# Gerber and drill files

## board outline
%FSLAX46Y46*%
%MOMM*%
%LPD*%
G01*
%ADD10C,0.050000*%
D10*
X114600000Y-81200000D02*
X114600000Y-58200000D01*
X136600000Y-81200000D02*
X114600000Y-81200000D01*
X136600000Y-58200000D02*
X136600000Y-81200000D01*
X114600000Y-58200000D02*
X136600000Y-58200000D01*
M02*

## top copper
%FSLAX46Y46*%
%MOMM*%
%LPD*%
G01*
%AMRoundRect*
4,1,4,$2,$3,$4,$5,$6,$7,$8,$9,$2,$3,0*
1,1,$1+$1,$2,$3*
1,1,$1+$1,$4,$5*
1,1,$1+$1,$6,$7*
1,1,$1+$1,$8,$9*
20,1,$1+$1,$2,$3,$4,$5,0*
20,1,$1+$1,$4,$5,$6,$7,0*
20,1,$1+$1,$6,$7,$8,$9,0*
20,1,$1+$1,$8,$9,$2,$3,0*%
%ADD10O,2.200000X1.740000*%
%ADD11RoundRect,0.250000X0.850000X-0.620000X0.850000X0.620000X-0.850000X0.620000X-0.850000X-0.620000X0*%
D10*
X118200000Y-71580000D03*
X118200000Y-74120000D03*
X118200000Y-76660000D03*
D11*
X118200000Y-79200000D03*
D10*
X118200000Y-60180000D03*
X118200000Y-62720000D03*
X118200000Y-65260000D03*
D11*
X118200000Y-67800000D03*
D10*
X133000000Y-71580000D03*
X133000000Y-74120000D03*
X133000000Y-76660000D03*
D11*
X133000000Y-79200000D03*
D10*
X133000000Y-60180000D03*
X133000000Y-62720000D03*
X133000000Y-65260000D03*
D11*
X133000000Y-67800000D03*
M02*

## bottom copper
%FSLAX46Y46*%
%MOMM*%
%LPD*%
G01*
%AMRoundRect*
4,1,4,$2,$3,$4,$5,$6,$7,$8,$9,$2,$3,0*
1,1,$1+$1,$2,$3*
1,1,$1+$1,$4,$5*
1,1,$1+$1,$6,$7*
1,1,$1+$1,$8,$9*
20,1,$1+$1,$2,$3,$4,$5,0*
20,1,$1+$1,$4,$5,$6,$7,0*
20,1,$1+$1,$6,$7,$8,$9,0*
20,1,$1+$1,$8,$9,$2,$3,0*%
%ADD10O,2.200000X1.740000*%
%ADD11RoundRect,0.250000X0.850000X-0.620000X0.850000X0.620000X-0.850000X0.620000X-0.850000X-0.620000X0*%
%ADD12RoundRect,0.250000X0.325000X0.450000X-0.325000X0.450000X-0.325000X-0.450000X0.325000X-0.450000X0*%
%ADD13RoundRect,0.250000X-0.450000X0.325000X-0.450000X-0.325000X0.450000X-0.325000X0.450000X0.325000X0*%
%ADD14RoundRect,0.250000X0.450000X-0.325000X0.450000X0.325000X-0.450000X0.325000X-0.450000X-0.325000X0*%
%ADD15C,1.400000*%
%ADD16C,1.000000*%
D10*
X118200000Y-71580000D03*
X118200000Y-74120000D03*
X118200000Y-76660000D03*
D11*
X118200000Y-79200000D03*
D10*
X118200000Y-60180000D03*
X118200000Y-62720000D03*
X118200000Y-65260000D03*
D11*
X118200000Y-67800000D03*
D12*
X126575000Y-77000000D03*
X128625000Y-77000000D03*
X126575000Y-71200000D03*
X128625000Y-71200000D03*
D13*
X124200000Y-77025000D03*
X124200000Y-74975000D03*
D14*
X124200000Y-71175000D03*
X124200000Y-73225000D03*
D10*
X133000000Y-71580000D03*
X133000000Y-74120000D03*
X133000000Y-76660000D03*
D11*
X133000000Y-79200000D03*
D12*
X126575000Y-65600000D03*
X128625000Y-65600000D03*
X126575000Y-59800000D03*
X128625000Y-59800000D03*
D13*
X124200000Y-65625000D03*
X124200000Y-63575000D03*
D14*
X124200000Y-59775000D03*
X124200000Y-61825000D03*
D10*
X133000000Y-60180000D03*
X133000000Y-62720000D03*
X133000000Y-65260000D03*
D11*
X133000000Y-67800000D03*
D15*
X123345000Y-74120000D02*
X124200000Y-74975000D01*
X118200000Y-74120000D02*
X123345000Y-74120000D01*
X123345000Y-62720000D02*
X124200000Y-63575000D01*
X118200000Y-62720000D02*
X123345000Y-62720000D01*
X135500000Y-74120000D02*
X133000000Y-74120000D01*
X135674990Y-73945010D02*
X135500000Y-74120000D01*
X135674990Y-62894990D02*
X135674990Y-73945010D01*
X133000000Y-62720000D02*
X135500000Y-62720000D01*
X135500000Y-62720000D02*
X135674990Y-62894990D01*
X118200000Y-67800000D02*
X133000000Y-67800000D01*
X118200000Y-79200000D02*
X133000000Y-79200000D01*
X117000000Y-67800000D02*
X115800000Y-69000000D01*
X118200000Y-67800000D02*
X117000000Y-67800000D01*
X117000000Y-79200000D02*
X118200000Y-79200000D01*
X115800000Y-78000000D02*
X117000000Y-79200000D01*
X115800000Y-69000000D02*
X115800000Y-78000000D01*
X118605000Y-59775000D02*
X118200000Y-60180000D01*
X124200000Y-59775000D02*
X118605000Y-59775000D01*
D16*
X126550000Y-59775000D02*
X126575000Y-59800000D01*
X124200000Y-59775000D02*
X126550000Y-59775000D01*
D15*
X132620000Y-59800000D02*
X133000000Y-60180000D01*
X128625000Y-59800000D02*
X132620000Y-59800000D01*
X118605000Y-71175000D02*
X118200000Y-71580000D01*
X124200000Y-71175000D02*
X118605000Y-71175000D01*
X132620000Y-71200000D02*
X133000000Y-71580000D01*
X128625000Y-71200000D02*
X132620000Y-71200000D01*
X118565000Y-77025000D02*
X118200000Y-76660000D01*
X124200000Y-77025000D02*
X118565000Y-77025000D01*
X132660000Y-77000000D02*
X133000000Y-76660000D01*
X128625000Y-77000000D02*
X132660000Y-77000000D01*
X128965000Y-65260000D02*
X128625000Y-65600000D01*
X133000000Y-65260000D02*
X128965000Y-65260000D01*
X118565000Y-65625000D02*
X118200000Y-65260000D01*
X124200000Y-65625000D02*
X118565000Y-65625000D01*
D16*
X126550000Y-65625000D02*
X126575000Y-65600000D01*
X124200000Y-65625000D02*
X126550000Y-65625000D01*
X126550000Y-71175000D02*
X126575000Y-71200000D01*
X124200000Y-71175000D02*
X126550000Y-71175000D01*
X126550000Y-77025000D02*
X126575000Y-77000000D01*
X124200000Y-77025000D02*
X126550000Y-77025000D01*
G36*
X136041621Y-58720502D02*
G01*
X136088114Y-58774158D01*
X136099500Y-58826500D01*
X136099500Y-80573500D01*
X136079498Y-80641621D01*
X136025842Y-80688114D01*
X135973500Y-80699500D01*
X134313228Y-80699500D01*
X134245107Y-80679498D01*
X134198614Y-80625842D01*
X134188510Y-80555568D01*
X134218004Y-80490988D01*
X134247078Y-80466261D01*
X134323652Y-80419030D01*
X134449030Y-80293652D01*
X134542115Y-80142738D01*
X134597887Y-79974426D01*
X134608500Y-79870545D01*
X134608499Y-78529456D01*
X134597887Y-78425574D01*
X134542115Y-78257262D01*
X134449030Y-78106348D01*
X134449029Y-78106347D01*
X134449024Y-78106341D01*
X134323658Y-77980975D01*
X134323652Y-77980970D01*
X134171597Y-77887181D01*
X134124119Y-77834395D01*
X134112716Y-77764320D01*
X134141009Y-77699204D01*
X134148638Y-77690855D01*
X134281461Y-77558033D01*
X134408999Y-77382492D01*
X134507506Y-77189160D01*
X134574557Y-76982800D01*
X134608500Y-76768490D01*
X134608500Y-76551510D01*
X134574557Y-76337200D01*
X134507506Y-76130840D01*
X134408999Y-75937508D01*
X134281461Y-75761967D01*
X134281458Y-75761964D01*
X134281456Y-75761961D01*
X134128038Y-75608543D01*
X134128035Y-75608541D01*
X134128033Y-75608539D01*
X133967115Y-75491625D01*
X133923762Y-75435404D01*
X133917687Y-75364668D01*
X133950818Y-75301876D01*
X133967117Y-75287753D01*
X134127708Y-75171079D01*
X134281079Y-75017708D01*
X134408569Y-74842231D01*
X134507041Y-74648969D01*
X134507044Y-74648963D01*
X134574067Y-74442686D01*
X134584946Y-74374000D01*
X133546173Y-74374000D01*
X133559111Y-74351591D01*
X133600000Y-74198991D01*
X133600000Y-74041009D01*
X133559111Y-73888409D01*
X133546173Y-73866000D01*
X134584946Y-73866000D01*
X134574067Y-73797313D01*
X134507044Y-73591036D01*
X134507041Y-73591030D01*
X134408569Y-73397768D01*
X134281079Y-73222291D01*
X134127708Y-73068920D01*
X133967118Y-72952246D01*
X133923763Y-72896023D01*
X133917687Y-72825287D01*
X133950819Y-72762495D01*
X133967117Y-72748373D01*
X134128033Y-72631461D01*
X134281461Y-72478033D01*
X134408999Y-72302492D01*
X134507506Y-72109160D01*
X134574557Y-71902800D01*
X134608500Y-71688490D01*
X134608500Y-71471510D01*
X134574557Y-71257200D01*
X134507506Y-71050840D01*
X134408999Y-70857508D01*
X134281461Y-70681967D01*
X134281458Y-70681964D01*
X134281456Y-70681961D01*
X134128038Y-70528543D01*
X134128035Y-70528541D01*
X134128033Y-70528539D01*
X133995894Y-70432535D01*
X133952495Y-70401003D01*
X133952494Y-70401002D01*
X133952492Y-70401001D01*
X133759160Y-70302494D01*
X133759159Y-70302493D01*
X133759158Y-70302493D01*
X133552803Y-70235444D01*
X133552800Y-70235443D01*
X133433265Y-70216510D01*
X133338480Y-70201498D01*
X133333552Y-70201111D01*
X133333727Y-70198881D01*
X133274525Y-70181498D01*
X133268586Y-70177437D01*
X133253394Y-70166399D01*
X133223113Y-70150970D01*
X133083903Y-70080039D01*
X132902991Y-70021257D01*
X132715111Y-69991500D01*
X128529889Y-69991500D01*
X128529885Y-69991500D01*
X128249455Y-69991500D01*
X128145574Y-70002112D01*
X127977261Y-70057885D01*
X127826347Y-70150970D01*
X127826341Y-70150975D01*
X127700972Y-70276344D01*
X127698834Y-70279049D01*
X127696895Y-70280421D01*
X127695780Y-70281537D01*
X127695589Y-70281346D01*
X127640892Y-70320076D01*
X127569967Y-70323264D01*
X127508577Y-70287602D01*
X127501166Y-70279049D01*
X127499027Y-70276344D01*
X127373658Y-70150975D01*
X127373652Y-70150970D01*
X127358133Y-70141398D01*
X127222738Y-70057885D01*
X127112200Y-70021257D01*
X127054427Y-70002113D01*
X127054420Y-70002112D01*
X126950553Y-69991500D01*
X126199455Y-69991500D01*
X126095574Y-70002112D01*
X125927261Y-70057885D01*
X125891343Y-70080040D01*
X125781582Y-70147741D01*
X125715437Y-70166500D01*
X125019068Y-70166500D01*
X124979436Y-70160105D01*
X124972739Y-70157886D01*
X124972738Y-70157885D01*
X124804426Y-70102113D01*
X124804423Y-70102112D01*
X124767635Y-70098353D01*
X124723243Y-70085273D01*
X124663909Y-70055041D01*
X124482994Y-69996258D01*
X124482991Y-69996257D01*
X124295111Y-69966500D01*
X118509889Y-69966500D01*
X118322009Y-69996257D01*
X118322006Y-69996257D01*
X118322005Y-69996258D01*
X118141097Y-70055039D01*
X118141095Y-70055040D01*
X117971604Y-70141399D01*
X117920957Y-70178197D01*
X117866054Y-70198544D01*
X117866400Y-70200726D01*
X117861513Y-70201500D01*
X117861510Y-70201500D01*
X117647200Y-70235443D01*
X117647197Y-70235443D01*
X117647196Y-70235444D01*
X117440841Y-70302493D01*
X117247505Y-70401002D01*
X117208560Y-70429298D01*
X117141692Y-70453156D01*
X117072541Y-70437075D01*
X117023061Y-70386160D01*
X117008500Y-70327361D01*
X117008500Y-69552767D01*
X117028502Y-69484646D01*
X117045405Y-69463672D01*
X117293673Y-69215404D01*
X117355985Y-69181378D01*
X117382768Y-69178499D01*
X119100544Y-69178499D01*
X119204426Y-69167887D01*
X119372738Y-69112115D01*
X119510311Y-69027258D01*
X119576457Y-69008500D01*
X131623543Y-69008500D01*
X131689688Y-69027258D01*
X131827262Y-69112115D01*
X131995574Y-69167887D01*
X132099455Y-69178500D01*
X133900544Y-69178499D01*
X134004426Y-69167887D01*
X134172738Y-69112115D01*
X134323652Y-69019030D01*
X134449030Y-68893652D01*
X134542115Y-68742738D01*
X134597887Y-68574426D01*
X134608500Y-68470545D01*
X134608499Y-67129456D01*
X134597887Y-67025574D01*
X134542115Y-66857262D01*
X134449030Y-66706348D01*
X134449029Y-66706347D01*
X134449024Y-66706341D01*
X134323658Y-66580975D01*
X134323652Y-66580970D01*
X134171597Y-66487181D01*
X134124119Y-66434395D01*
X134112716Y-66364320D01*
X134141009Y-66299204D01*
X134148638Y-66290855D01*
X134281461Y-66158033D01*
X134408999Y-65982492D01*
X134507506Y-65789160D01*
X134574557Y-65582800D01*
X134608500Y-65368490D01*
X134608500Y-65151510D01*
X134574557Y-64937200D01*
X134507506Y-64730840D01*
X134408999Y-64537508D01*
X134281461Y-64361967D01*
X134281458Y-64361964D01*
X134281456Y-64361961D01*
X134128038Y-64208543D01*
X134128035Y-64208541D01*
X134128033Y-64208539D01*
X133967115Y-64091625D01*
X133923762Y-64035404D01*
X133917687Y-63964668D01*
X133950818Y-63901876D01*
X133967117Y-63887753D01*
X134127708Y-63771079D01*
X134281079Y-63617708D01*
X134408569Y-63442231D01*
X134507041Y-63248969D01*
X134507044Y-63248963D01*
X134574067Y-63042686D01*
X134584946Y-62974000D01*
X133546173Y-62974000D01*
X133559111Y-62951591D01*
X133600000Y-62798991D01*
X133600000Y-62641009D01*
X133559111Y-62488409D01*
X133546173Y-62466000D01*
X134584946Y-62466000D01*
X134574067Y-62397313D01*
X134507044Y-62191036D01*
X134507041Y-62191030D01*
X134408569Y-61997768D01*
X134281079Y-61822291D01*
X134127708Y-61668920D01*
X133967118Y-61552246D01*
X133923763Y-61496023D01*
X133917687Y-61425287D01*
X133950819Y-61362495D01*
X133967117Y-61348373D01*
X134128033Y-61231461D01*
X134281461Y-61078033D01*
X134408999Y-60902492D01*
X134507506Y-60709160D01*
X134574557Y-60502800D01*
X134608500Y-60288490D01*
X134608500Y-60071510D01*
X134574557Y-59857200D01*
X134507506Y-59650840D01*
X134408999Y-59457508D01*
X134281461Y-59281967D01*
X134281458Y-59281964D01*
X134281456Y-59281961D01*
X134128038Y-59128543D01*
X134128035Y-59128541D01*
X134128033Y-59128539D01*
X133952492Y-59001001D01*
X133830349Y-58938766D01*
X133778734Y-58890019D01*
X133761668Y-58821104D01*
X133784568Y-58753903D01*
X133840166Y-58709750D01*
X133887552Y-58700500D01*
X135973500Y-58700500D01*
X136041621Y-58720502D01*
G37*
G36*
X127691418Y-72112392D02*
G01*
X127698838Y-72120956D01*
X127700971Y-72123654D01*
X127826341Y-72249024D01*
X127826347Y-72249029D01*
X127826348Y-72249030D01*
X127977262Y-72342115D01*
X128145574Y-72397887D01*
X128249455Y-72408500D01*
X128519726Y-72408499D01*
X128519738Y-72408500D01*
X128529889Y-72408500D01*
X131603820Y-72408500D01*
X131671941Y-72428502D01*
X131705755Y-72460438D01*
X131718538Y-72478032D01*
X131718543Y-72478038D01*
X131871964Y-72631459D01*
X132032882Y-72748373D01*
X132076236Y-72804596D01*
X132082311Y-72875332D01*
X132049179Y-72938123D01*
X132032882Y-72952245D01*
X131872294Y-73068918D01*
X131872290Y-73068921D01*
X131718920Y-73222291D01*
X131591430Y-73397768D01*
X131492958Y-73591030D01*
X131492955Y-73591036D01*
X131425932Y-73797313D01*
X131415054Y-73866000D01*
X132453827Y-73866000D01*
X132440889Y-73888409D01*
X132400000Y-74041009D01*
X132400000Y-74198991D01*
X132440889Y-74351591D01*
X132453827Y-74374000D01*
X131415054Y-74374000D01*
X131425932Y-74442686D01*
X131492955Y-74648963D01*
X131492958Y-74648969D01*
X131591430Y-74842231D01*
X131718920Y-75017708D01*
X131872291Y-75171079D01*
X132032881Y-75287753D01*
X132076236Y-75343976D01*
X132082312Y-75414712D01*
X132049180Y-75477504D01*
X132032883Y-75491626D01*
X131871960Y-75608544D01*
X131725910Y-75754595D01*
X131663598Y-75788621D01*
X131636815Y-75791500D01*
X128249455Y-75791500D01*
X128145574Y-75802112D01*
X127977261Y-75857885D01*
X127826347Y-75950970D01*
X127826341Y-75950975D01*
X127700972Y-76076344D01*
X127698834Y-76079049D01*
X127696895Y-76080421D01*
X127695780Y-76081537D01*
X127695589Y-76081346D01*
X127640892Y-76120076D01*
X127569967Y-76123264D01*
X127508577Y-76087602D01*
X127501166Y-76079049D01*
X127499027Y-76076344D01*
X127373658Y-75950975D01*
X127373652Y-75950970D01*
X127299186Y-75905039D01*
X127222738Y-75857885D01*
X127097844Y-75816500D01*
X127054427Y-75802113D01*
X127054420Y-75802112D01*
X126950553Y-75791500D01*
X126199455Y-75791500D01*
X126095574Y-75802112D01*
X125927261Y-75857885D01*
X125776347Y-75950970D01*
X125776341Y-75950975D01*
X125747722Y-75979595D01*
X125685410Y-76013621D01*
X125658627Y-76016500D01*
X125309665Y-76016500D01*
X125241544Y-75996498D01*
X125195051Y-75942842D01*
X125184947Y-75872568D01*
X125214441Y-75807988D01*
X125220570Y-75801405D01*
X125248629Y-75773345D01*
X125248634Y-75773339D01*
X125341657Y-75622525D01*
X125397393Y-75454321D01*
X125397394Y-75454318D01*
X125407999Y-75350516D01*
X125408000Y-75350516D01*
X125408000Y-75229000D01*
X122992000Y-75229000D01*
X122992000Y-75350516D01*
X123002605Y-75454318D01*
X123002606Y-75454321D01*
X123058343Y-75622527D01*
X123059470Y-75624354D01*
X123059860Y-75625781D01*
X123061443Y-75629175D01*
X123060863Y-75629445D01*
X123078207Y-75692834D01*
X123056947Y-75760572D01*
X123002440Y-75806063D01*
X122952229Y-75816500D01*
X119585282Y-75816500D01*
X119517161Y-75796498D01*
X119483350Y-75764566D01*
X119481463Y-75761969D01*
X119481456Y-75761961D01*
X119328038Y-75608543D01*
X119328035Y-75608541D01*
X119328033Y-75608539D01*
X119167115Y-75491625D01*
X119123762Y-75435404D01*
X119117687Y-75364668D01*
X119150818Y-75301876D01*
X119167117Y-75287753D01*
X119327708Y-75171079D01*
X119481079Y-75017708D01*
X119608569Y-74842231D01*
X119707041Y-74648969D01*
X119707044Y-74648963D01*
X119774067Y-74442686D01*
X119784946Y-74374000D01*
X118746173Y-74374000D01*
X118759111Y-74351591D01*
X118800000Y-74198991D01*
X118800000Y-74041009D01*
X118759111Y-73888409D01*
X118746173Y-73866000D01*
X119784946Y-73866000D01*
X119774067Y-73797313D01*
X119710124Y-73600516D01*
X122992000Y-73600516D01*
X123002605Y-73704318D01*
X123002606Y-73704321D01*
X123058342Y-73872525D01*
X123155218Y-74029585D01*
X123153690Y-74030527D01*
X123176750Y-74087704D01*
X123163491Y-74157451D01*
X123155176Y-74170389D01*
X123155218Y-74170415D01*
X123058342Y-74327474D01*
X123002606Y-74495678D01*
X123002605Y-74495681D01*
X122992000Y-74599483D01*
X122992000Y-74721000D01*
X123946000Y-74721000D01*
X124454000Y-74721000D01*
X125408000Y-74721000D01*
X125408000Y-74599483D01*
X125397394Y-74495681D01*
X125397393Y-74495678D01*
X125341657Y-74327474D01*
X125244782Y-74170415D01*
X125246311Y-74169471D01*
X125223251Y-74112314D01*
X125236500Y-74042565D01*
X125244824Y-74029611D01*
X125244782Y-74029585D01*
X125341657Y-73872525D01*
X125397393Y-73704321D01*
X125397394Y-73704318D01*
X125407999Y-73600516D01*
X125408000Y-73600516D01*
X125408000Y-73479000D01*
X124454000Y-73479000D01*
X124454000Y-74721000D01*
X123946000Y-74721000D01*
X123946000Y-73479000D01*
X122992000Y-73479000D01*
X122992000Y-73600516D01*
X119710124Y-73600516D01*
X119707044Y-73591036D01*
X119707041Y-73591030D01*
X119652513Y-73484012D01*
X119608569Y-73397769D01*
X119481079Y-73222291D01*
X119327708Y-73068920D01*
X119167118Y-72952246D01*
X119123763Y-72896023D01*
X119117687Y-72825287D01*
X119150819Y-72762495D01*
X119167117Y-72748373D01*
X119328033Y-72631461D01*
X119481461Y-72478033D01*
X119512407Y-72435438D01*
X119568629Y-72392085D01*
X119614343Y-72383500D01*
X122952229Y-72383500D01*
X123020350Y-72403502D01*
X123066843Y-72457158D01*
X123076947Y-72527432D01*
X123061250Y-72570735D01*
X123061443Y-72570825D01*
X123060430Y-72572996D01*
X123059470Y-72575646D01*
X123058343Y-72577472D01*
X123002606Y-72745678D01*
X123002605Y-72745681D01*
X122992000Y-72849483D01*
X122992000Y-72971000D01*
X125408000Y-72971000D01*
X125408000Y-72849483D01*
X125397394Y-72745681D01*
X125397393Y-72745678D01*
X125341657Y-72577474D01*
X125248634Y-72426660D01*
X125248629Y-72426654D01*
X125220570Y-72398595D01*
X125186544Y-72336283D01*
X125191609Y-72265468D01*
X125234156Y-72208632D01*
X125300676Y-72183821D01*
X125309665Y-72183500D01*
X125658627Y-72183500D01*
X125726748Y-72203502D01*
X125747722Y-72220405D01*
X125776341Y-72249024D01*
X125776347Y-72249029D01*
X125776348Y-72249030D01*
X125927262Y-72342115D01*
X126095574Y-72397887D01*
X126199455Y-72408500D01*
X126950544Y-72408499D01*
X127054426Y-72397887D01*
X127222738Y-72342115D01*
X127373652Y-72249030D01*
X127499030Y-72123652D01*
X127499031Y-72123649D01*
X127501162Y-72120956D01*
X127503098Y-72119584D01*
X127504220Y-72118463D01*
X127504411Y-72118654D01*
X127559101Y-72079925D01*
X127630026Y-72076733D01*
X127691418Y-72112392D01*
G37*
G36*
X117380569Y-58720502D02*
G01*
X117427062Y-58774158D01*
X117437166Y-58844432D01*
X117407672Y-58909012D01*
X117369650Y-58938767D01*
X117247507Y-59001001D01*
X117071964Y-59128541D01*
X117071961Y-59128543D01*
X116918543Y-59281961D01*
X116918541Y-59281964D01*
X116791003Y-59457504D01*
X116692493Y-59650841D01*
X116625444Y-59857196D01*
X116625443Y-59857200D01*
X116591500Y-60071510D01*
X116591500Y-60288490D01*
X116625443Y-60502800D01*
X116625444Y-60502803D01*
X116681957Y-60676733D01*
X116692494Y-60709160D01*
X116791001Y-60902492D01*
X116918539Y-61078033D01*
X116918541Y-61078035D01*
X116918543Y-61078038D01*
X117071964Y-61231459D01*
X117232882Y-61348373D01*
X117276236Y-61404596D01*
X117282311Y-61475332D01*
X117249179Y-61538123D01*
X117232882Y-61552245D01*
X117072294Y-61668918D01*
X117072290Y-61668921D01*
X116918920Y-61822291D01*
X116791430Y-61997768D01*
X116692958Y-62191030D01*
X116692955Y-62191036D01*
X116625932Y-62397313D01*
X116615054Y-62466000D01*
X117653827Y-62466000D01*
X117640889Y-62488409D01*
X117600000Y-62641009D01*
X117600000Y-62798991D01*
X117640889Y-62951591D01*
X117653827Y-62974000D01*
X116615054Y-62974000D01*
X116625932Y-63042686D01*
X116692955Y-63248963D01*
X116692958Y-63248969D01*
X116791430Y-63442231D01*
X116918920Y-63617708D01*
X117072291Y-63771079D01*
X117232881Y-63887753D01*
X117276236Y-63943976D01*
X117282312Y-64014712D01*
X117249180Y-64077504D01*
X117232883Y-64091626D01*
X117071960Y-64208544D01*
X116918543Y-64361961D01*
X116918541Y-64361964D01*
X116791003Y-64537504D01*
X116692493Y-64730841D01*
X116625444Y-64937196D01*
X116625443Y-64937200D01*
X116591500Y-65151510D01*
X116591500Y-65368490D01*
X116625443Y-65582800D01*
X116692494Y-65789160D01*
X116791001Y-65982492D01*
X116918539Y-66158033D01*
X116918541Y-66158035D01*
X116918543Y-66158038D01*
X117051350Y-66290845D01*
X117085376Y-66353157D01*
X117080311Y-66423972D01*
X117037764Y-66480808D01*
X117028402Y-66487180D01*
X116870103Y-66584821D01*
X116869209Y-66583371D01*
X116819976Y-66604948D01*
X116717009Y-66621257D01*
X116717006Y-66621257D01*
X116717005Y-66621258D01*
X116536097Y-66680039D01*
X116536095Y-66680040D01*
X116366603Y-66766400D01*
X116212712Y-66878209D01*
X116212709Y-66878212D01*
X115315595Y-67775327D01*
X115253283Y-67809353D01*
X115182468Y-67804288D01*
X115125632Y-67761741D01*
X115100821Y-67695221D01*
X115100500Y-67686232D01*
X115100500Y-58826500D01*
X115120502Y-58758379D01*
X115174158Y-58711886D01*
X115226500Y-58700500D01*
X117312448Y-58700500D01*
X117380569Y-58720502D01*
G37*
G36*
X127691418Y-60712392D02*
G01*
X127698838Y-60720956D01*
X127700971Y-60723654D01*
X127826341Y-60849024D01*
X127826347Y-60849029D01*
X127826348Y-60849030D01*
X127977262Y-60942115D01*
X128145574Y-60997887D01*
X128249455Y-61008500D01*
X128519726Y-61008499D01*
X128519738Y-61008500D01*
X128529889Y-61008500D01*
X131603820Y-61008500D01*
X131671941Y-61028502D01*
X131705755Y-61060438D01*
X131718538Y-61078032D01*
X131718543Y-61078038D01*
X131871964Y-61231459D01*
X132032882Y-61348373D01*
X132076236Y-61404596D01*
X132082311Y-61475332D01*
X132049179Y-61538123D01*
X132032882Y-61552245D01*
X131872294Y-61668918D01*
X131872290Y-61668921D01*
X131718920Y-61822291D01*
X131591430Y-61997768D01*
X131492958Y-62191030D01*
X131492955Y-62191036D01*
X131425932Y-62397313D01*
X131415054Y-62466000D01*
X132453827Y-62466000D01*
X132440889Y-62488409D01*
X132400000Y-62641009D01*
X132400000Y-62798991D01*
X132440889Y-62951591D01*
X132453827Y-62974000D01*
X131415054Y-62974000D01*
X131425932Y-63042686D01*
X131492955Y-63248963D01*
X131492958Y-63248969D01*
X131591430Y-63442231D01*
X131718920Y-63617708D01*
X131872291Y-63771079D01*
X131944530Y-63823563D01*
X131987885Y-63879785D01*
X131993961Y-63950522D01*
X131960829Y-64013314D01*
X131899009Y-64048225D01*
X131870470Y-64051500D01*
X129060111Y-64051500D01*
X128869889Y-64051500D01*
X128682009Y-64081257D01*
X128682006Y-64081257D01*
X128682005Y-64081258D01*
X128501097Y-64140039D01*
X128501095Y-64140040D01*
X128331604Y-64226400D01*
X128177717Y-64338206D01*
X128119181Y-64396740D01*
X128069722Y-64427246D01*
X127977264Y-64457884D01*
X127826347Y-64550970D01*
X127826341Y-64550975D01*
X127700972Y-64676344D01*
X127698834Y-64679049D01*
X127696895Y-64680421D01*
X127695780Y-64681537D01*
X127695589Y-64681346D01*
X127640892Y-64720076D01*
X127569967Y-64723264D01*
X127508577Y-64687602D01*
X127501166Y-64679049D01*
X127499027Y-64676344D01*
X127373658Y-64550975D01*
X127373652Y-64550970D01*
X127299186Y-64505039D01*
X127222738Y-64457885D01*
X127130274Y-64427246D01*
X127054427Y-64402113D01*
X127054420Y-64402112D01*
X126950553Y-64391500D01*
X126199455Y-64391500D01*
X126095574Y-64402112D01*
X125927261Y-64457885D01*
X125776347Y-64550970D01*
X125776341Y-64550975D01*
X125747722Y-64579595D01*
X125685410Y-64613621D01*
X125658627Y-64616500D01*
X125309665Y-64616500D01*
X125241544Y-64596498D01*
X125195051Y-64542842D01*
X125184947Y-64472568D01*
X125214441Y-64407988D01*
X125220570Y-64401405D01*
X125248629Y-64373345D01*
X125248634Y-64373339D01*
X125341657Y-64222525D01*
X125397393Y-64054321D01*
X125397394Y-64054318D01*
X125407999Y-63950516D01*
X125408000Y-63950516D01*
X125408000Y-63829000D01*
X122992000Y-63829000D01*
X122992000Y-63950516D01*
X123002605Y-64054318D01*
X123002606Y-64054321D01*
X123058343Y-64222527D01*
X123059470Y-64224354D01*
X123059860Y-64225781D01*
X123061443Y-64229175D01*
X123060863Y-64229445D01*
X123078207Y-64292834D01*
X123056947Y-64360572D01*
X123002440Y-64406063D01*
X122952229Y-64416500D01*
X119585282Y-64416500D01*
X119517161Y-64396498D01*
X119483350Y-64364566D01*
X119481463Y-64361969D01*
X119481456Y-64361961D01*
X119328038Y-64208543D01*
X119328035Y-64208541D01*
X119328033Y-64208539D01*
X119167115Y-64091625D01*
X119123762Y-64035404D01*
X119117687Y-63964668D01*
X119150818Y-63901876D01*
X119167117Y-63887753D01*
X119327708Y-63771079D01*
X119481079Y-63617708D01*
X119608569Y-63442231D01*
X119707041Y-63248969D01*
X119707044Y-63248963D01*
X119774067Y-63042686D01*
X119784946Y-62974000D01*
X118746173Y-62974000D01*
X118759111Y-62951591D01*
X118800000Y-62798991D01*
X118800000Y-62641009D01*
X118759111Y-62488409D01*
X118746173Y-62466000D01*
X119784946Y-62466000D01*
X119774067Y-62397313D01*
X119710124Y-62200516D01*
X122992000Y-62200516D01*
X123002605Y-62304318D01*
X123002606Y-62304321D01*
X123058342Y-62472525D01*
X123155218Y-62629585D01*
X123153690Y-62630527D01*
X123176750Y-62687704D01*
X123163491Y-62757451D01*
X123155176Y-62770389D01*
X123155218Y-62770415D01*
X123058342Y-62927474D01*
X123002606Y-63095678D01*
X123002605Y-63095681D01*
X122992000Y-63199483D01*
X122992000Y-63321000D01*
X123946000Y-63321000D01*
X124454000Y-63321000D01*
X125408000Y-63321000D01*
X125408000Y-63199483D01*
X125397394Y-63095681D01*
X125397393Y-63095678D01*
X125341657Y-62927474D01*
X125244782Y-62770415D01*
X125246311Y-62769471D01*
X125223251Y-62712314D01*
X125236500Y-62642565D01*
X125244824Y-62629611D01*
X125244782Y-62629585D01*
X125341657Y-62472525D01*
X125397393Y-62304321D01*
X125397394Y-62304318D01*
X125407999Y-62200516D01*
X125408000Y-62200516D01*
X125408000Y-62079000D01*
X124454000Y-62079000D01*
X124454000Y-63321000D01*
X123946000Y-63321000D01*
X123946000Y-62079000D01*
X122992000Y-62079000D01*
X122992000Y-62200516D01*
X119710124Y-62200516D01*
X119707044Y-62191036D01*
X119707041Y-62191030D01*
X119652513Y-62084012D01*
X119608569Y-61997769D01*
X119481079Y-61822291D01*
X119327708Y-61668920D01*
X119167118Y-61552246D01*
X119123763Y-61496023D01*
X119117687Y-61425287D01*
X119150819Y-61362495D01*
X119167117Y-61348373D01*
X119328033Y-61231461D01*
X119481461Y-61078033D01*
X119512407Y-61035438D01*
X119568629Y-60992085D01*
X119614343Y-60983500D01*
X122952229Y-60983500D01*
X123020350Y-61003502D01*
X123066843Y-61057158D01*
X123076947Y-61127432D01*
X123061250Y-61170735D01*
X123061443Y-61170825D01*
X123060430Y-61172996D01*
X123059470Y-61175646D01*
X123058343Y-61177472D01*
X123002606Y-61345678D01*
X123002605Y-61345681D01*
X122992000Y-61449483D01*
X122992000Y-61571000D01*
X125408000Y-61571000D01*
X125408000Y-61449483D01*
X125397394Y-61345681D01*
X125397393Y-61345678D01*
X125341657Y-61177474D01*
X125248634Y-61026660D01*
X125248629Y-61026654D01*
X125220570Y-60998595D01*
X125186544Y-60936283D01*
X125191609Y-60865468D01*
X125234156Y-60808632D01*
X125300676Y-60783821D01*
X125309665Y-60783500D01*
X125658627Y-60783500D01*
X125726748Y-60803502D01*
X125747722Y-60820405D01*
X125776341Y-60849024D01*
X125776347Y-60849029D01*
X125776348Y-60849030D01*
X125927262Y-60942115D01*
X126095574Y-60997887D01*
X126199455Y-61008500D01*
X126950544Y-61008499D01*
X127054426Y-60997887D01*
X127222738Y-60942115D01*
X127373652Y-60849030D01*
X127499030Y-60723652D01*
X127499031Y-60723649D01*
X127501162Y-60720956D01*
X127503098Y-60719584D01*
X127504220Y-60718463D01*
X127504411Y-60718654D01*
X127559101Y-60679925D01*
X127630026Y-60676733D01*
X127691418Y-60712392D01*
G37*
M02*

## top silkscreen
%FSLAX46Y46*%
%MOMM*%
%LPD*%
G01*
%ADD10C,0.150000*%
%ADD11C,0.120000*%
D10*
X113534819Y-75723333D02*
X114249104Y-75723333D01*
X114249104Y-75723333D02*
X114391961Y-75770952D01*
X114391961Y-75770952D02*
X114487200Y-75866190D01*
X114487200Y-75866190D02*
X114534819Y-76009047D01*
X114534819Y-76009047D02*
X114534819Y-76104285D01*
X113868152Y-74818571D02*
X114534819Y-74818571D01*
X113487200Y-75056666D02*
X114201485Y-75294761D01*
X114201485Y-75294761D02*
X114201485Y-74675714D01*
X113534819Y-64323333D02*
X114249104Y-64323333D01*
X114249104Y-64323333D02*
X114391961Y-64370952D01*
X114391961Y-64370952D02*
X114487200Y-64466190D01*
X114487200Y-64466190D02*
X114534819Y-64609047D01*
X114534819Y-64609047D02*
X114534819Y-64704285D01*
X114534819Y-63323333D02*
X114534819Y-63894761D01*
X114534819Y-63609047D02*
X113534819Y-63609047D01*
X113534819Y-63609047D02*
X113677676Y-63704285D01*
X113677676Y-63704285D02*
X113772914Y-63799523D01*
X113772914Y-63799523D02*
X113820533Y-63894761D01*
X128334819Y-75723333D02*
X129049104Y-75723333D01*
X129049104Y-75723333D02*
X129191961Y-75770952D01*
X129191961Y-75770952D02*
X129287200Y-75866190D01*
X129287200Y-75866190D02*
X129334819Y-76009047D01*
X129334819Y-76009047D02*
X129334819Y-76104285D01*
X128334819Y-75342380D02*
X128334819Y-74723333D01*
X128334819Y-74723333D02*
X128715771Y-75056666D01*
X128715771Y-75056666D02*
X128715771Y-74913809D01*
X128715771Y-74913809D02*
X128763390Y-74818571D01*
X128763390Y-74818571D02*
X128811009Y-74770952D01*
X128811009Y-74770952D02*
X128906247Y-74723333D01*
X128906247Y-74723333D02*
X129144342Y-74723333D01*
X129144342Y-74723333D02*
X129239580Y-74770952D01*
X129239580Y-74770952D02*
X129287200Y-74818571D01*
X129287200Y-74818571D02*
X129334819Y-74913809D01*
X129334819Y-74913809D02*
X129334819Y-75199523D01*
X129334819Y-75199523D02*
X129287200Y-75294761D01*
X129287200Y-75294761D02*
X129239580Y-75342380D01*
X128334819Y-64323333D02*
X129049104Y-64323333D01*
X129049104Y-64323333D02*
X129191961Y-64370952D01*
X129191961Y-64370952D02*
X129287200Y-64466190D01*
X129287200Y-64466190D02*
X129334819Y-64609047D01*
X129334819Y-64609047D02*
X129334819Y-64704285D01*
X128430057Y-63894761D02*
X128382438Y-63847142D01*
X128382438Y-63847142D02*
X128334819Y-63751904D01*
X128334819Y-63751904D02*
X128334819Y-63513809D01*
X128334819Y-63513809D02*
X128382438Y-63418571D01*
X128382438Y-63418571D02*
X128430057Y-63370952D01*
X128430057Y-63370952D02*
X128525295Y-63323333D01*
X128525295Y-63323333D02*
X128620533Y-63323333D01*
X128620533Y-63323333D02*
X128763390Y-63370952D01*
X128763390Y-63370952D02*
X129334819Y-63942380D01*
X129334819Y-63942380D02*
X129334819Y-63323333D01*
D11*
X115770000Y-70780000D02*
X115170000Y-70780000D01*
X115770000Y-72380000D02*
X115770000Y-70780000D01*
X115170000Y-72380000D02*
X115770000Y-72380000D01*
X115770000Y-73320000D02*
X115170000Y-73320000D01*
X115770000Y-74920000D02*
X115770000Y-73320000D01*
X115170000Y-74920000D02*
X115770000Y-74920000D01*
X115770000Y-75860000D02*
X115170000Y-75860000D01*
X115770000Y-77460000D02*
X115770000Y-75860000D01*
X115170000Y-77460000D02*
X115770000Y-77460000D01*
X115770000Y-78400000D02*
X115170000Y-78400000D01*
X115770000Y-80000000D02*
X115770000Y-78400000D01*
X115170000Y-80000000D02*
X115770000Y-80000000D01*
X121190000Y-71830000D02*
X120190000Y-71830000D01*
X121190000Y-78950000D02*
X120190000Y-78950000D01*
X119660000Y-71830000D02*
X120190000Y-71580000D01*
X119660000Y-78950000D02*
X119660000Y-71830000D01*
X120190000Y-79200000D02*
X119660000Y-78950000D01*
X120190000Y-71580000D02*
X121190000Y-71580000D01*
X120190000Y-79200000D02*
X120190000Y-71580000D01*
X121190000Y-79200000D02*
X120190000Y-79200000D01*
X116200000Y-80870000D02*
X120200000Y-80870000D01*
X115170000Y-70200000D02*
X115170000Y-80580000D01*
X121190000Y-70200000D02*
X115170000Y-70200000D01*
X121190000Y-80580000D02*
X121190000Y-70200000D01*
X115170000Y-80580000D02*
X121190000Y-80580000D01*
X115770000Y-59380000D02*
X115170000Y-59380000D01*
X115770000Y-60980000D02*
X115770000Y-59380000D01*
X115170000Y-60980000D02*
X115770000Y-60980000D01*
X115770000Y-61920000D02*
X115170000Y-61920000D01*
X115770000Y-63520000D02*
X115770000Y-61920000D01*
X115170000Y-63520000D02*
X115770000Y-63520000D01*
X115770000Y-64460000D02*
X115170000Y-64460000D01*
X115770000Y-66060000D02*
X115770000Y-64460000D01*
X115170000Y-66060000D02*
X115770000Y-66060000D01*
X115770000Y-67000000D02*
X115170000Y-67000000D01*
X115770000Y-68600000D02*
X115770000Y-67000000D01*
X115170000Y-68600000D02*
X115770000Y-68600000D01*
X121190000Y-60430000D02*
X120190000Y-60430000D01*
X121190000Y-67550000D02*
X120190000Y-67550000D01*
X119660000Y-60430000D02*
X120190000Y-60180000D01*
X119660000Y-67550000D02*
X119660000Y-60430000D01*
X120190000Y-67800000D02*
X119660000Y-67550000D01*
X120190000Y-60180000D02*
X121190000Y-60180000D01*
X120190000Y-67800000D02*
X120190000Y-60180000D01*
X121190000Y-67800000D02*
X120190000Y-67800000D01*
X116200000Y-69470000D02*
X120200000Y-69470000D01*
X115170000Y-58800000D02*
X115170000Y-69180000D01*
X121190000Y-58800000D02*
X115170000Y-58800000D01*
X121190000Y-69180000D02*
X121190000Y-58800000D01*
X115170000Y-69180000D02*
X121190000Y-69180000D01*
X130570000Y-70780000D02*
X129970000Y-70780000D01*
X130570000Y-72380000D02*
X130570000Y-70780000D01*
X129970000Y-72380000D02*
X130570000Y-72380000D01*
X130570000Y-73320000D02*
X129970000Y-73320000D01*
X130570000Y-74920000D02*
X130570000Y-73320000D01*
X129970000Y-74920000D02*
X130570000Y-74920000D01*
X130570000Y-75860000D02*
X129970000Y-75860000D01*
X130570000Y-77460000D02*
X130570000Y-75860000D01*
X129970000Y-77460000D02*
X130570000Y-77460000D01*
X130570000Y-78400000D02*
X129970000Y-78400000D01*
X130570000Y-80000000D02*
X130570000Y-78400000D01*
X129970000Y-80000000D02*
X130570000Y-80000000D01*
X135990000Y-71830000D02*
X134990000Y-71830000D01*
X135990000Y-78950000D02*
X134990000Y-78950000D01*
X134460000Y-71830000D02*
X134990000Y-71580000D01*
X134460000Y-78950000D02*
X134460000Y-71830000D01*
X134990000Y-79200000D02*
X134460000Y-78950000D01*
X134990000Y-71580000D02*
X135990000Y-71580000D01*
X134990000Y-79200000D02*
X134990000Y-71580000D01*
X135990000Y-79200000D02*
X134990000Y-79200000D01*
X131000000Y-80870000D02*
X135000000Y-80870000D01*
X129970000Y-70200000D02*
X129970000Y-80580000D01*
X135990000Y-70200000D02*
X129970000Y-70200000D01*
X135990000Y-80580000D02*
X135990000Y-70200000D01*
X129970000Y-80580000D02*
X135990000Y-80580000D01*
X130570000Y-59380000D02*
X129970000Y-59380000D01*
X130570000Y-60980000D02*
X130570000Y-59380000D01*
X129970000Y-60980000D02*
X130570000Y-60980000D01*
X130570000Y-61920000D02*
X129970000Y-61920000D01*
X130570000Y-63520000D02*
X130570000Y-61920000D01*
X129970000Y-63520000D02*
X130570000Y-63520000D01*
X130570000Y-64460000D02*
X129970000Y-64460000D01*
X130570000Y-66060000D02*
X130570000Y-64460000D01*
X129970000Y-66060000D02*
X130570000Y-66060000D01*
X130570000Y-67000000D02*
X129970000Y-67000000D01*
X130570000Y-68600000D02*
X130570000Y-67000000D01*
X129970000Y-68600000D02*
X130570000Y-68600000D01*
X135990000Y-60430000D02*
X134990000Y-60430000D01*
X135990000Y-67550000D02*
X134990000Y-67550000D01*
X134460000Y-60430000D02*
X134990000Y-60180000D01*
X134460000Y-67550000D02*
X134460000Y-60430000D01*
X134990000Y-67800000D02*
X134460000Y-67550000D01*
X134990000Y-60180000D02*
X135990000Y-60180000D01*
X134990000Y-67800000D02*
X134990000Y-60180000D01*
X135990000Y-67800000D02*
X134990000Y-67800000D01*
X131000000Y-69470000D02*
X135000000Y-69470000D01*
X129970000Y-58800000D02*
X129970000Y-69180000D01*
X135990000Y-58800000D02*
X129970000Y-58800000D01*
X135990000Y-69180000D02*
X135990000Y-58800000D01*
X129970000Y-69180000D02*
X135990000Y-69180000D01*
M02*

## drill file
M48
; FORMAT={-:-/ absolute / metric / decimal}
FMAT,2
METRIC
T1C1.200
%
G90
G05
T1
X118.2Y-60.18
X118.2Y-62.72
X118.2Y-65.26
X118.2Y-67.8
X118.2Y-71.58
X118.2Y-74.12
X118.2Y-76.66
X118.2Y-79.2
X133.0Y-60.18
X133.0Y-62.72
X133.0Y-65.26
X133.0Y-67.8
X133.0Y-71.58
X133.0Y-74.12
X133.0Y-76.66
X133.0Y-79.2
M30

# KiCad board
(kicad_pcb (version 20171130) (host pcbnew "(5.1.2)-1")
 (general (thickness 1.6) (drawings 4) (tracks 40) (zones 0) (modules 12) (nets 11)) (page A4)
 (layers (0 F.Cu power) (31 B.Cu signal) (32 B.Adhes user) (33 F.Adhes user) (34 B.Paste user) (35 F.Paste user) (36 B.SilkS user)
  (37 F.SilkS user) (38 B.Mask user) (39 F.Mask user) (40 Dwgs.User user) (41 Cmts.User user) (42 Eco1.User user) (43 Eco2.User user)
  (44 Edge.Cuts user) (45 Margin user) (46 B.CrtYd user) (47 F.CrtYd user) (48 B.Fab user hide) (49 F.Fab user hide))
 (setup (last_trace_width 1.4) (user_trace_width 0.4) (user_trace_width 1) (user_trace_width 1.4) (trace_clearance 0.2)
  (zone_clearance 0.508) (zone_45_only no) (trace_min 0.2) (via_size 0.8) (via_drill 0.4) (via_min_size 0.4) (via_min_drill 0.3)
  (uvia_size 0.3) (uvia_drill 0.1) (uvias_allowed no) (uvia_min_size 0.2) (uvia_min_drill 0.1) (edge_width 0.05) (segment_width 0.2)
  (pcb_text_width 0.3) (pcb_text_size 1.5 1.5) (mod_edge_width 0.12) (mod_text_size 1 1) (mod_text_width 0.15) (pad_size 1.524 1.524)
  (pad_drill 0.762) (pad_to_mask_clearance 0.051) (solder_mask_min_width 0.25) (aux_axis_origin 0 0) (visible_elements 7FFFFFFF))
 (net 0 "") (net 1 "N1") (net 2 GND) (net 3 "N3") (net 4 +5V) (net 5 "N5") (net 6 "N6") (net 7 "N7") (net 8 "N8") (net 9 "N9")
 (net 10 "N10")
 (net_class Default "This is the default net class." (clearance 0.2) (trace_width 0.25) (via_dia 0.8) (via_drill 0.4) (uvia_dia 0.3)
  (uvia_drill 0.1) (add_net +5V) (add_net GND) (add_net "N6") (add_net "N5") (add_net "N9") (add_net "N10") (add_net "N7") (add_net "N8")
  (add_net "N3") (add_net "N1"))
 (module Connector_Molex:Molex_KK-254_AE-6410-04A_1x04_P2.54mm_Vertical (layer F.Cu) (at 118.2 79.2 90)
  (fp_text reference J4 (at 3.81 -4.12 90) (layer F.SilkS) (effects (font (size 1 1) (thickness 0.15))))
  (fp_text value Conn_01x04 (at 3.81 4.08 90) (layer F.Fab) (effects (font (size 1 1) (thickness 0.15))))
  (fp_line (start 8.42 -2.43) (end 8.42 -3.03) (layer F.SilkS) (width 0.12))
  (fp_line (start 6.82 -2.43) (end 8.42 -2.43) (layer F.SilkS) (width 0.12))
  (fp_line (start 6.82 -3.03) (end 6.82 -2.43) (layer F.SilkS) (width 0.12))
  (fp_line (start 5.88 -2.43) (end 5.88 -3.03) (layer F.SilkS) (width 0.12))
  (fp_line (start 4.28 -2.43) (end 5.88 -2.43) (layer F.SilkS) (width 0.12))
  (fp_line (start 4.28 -3.03) (end 4.28 -2.43) (layer F.SilkS) (width 0.12))
  (fp_line (start 3.34 -2.43) (end 3.34 -3.03) (layer F.SilkS) (width 0.12))
  (fp_line (start 1.74 -2.43) (end 3.34 -2.43) (layer F.SilkS) (width 0.12))
  (fp_line (start 1.74 -3.03) (end 1.74 -2.43) (layer F.SilkS) (width 0.12))
  (fp_line (start 0.8 -2.43) (end 0.8 -3.03) (layer F.SilkS) (width 0.12))
  (fp_line (start -0.8 -2.43) (end 0.8 -2.43) (layer F.SilkS) (width 0.12))
  (fp_line (start -0.8 -3.03) (end -0.8 -2.43) (layer F.SilkS) (width 0.12))
  (fp_line (start 7.37 2.99) (end 7.37 1.99) (layer F.SilkS) (width 0.12))
  (fp_line (start 0.25 2.99) (end 0.25 1.99) (layer F.SilkS) (width 0.12))
  (fp_line (start 7.37 1.46) (end 7.62 1.99) (layer F.SilkS) (width 0.12))
  (fp_line (start 0.25 1.46) (end 7.37 1.46) (layer F.SilkS) (width 0.12))
  (fp_line (start 0 1.99) (end 0.25 1.46) (layer F.SilkS) (width 0.12))
  (fp_line (start 7.62 1.99) (end 7.62 2.99) (layer F.SilkS) (width 0.12))
  (fp_line (start 0 1.99) (end 7.62 1.99) (layer F.SilkS) (width 0.12))
  (fp_line (start 0 2.99) (end 0 1.99) (layer F.SilkS) (width 0.12))
  (fp_line (start -1.67 -2) (end -1.67 2) (layer F.SilkS) (width 0.12))
  (fp_line (start 9 -3.03) (end -1.38 -3.03) (layer F.SilkS) (width 0.12))
  (fp_line (start 9 2.99) (end 9 -3.03) (layer F.SilkS) (width 0.12))
  (fp_line (start -1.38 2.99) (end 9 2.99) (layer F.SilkS) (width 0.12))
  (fp_line (start -1.38 -3.03) (end -1.38 2.99) (layer F.SilkS) (width 0.12))
  (pad 4 thru_hole oval (at 7.62 0 90) (size 1.74 2.2) (drill 1.2) (layers *.Cu *.Mask) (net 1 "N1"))
  (pad 3 thru_hole oval (at 5.08 0 90) (size 1.74 2.2) (drill 1.2) (layers *.Cu *.Mask) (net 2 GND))
  (pad 2 thru_hole oval (at 2.54 0 90) (size 1.74 2.2) (drill 1.2) (layers *.Cu *.Mask) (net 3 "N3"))
  (pad 1 thru_hole roundrect (at 0 0 90) (size 1.74 2.2) (drill 1.2) (layers *.Cu *.Mask) (roundrect_rratio 0.143678) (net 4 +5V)))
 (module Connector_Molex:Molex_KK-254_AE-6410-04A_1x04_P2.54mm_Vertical (layer F.Cu) (at 118.2 67.8 90)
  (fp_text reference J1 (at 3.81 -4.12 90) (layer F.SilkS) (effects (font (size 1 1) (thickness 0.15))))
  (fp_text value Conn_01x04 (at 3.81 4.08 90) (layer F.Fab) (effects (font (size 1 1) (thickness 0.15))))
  (fp_line (start 8.42 -2.43) (end 8.42 -3.03) (layer F.SilkS) (width 0.12))
  (fp_line (start 6.82 -2.43) (end 8.42 -2.43) (layer F.SilkS) (width 0.12))
  (fp_line (start 6.82 -3.03) (end 6.82 -2.43) (layer F.SilkS) (width 0.12))
  (fp_line (start 5.88 -2.43) (end 5.88 -3.03) (layer F.SilkS) (width 0.12))
  (fp_line (start 4.28 -2.43) (end 5.88 -2.43) (layer F.SilkS) (width 0.12))
  (fp_line (start 4.28 -3.03) (end 4.28 -2.43) (layer F.SilkS) (width 0.12))
  (fp_line (start 3.34 -2.43) (end 3.34 -3.03) (layer F.SilkS) (width 0.12))
  (fp_line (start 1.74 -2.43) (end 3.34 -2.43) (layer F.SilkS) (width 0.12))
  (fp_line (start 1.74 -3.03) (end 1.74 -2.43) (layer F.SilkS) (width 0.12))
  (fp_line (start 0.8 -2.43) (end 0.8 -3.03) (layer F.SilkS) (width 0.12))
  (fp_line (start -0.8 -2.43) (end 0.8 -2.43) (layer F.SilkS) (width 0.12))
  (fp_line (start -0.8 -3.03) (end -0.8 -2.43) (layer F.SilkS) (width 0.12))
  (fp_line (start 7.37 2.99) (end 7.37 1.99) (layer F.SilkS) (width 0.12))
  (fp_line (start 0.25 2.99) (end 0.25 1.99) (layer F.SilkS) (width 0.12))
  (fp_line (start 7.37 1.46) (end 7.62 1.99) (layer F.SilkS) (width 0.12))
  (fp_line (start 0.25 1.46) (end 7.37 1.46) (layer F.SilkS) (width 0.12))
  (fp_line (start 0 1.99) (end 0.25 1.46) (layer F.SilkS) (width 0.12))
  (fp_line (start 7.62 1.99) (end 7.62 2.99) (layer F.SilkS) (width 0.12))
  (fp_line (start 0 1.99) (end 7.62 1.99) (layer F.SilkS) (width 0.12))
  (fp_line (start 0 2.99) (end 0 1.99) (layer F.SilkS) (width 0.12))
  (fp_line (start -1.67 -2) (end -1.67 2) (layer F.SilkS) (width 0.12))
  (fp_line (start 9 -3.03) (end -1.38 -3.03) (layer F.SilkS) (width 0.12))
  (fp_line (start 9 2.99) (end 9 -3.03) (layer F.SilkS) (width 0.12))
  (fp_line (start -1.38 2.99) (end 9 2.99) (layer F.SilkS) (width 0.12))
  (fp_line (start -1.38 -3.03) (end -1.38 2.99) (layer F.SilkS) (width 0.12))
  (pad 4 thru_hole oval (at 7.62 0 90) (size 1.74 2.2) (drill 1.2) (layers *.Cu *.Mask) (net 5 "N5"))
  (pad 3 thru_hole oval (at 5.08 0 90) (size 1.74 2.2) (drill 1.2) (layers *.Cu *.Mask) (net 2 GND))
  (pad 2 thru_hole oval (at 2.54 0 90) (size 1.74 2.2) (drill 1.2) (layers *.Cu *.Mask) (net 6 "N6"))
  (pad 1 thru_hole roundrect (at 0 0 90) (size 1.74 2.2) (drill 1.2) (layers *.Cu *.Mask) (roundrect_rratio 0.143678) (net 4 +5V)))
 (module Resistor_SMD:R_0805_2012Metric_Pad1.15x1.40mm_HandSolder (layer B.Cu) (at 127.6 77 180)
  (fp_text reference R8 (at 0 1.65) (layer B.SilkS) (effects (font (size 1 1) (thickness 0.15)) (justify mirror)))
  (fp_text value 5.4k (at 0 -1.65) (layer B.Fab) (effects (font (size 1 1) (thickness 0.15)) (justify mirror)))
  (pad 2 smd roundrect (at 1.025 0 180) (size 1.15 1.4) (layers B.Cu B.Paste B.Mask) (roundrect_rratio 0.217391) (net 3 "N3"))
  (pad 1 smd roundrect (at -1.025 0 180) (size 1.15 1.4) (layers B.Cu B.Paste B.Mask) (roundrect_rratio 0.217391) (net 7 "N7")))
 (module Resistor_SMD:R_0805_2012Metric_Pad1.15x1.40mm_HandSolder (layer B.Cu) (at 127.6 71.2 180)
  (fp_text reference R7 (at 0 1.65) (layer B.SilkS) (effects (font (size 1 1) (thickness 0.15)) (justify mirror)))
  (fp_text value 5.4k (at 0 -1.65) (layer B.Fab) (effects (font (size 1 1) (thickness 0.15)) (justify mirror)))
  (pad 2 smd roundrect (at 1.025 0 180) (size 1.15 1.4) (layers B.Cu B.Paste B.Mask) (roundrect_rratio 0.217391) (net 1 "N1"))
  (pad 1 smd roundrect (at -1.025 0 180) (size 1.15 1.4) (layers B.Cu B.Paste B.Mask) (roundrect_rratio 0.217391) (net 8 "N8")))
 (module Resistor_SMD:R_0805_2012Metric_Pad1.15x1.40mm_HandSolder (layer B.Cu) (at 124.2 76 270)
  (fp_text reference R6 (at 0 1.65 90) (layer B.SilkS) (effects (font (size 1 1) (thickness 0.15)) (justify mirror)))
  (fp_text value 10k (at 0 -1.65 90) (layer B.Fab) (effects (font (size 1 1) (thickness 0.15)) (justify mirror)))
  (pad 2 smd roundrect (at 1.025 0 270) (size 1.15 1.4) (layers B.Cu B.Paste B.Mask) (roundrect_rratio 0.217391) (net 3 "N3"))
  (pad 1 smd roundrect (at -1.025 0 270) (size 1.15 1.4) (layers B.Cu B.Paste B.Mask) (roundrect_rratio 0.217391) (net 2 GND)))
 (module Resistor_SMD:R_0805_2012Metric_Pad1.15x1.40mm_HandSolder (layer B.Cu) (at 124.2 72.2 90)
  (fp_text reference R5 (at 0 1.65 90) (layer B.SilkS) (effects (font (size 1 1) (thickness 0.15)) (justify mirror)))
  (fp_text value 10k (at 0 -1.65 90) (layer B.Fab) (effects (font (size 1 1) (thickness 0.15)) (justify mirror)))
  (pad 2 smd roundrect (at 1.025 0 90) (size 1.15 1.4) (layers B.Cu B.Paste B.Mask) (roundrect_rratio 0.217391) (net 1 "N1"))
  (pad 1 smd roundrect (at -1.025 0 90) (size 1.15 1.4) (layers B.Cu B.Paste B.Mask) (roundrect_rratio 0.217391) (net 2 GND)))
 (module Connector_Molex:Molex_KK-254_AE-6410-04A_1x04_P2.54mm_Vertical (layer F.Cu) (at 133 79.2 90)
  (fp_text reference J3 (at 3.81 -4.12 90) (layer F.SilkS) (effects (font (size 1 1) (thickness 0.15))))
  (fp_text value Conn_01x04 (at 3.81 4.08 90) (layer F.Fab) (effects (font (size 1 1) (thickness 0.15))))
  (fp_line (start 8.42 -2.43) (end 8.42 -3.03) (layer F.SilkS) (width 0.12))
  (fp_line (start 6.82 -2.43) (end 8.42 -2.43) (layer F.SilkS) (width 0.12))
  (fp_line (start 6.82 -3.03) (end 6.82 -2.43) (layer F.SilkS) (width 0.12))
  (fp_line (start 5.88 -2.43) (end 5.88 -3.03) (layer F.SilkS) (width 0.12))
  (fp_line (start 4.28 -2.43) (end 5.88 -2.43) (layer F.SilkS) (width 0.12))
  (fp_line (start 4.28 -3.03) (end 4.28 -2.43) (layer F.SilkS) (width 0.12))
  (fp_line (start 3.34 -2.43) (end 3.34 -3.03) (layer F.SilkS) (width 0.12))
  (fp_line (start 1.74 -2.43) (end 3.34 -2.43) (layer F.SilkS) (width 0.12))
  (fp_line (start 1.74 -3.03) (end 1.74 -2.43) (layer F.SilkS) (width 0.12))
  (fp_line (start 0.8 -2.43) (end 0.8 -3.03) (layer F.SilkS) (width 0.12))
  (fp_line (start -0.8 -2.43) (end 0.8 -2.43) (layer F.SilkS) (width 0.12))
  (fp_line (start -0.8 -3.03) (end -0.8 -2.43) (layer F.SilkS) (width 0.12))
  (fp_line (start 7.37 2.99) (end 7.37 1.99) (layer F.SilkS) (width 0.12))
  (fp_line (start 0.25 2.99) (end 0.25 1.99) (layer F.SilkS) (width 0.12))
  (fp_line (start 7.37 1.46) (end 7.62 1.99) (layer F.SilkS) (width 0.12))
  (fp_line (start 0.25 1.46) (end 7.37 1.46) (layer F.SilkS) (width 0.12))
  (fp_line (start 0 1.99) (end 0.25 1.46) (layer F.SilkS) (width 0.12))
  (fp_line (start 7.62 1.99) (end 7.62 2.99) (layer F.SilkS) (width 0.12))
  (fp_line (start 0 1.99) (end 7.62 1.99) (layer F.SilkS) (width 0.12))
  (fp_line (start 0 2.99) (end 0 1.99) (layer F.SilkS) (width 0.12))
  (fp_line (start -1.67 -2) (end -1.67 2) (layer F.SilkS) (width 0.12))
  (fp_line (start 9 -3.03) (end -1.38 -3.03) (layer F.SilkS) (width 0.12))
  (fp_line (start 9 2.99) (end 9 -3.03) (layer F.SilkS) (width 0.12))
  (fp_line (start -1.38 2.99) (end 9 2.99) (layer F.SilkS) (width 0.12))
  (fp_line (start -1.38 -3.03) (end -1.38 2.99) (layer F.SilkS) (width 0.12))
  (pad 4 thru_hole oval (at 7.62 0 90) (size 1.74 2.2) (drill 1.2) (layers *.Cu *.Mask) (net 8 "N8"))
  (pad 3 thru_hole oval (at 5.08 0 90) (size 1.74 2.2) (drill 1.2) (layers *.Cu *.Mask) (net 2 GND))
  (pad 2 thru_hole oval (at 2.54 0 90) (size 1.74 2.2) (drill 1.2) (layers *.Cu *.Mask) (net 7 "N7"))
  (pad 1 thru_hole roundrect (at 0 0 90) (size 1.74 2.2) (drill 1.2) (layers *.Cu *.Mask) (roundrect_rratio 0.143678) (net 4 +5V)))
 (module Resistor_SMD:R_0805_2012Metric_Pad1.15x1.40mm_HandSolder (layer B.Cu) (at 127.6 65.6 180)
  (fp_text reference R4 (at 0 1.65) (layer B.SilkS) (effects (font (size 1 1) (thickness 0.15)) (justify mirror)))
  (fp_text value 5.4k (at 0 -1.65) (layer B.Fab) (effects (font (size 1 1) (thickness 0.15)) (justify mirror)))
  (pad 2 smd roundrect (at 1.025 0 180) (size 1.15 1.4) (layers B.Cu B.Paste B.Mask) (roundrect_rratio 0.217391) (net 6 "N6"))
  (pad 1 smd roundrect (at -1.025 0 180) (size 1.15 1.4) (layers B.Cu B.Paste B.Mask) (roundrect_rratio 0.217391) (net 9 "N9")))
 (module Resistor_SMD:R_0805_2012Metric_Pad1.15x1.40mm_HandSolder (layer B.Cu) (at 127.6 59.8 180)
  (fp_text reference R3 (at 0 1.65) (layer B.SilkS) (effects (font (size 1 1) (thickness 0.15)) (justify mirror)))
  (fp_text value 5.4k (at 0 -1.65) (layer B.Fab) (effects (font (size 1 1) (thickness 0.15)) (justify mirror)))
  (pad 2 smd roundrect (at 1.025 0 180) (size 1.15 1.4) (layers B.Cu B.Paste B.Mask) (roundrect_rratio 0.217391) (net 5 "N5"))
  (pad 1 smd roundrect (at -1.025 0 180) (size 1.15 1.4) (layers B.Cu B.Paste B.Mask) (roundrect_rratio 0.217391) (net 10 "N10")))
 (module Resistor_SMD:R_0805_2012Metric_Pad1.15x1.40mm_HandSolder (layer B.Cu) (at 124.2 64.6 270)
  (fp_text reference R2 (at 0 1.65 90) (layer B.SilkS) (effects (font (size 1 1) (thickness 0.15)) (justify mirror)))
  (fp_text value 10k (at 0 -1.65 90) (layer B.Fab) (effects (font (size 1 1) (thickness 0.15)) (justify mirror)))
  (pad 2 smd roundrect (at 1.025 0 270) (size 1.15 1.4) (layers B.Cu B.Paste B.Mask) (roundrect_rratio 0.217391) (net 6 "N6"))
  (pad 1 smd roundrect (at -1.025 0 270) (size 1.15 1.4) (layers B.Cu B.Paste B.Mask) (roundrect_rratio 0.217391) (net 2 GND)))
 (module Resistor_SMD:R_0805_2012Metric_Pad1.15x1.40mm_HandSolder (layer B.Cu) (at 124.2 60.8 90)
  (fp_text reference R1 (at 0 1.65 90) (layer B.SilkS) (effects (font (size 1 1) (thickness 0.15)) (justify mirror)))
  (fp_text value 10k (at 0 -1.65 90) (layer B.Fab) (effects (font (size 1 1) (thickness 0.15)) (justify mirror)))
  (pad 2 smd roundrect (at 1.025 0 90) (size 1.15 1.4) (layers B.Cu B.Paste B.Mask) (roundrect_rratio 0.217391) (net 5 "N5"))
  (pad 1 smd roundrect (at -1.025 0 90) (size 1.15 1.4) (layers B.Cu B.Paste B.Mask) (roundrect_rratio 0.217391) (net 2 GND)))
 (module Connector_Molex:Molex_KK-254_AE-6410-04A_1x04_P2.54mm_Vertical (layer F.Cu) (at 133 67.8 90)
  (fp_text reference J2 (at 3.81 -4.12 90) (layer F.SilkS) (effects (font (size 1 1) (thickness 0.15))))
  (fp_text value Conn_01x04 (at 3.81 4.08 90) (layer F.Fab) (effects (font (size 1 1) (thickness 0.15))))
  (fp_line (start 8.42 -2.43) (end 8.42 -3.03) (layer F.SilkS) (width 0.12))
  (fp_line (start 6.82 -2.43) (end 8.42 -2.43) (layer F.SilkS) (width 0.12))
  (fp_line (start 6.82 -3.03) (end 6.82 -2.43) (layer F.SilkS) (width 0.12))
  (fp_line (start 5.88 -2.43) (end 5.88 -3.03) (layer F.SilkS) (width 0.12))
  (fp_line (start 4.28 -2.43) (end 5.88 -2.43) (layer F.SilkS) (width 0.12))
  (fp_line (start 4.28 -3.03) (end 4.28 -2.43) (layer F.SilkS) (width 0.12))
  (fp_line (start 3.34 -2.43) (end 3.34 -3.03) (layer F.SilkS) (width 0.12))
  (fp_line (start 1.74 -2.43) (end 3.34 -2.43) (layer F.SilkS) (width 0.12))
  (fp_line (start 1.74 -3.03) (end 1.74 -2.43) (layer F.SilkS) (width 0.12))
  (fp_line (start 0.8 -2.43) (end 0.8 -3.03) (layer F.SilkS) (width 0.12))
  (fp_line (start -0.8 -2.43) (end 0.8 -2.43) (layer F.SilkS) (width 0.12))
  (fp_line (start -0.8 -3.03) (end -0.8 -2.43) (layer F.SilkS) (width 0.12))
  (fp_line (start 7.37 2.99) (end 7.37 1.99) (layer F.SilkS) (width 0.12))
  (fp_line (start 0.25 2.99) (end 0.25 1.99) (layer F.SilkS) (width 0.12))
  (fp_line (start 7.37 1.46) (end 7.62 1.99) (layer F.SilkS) (width 0.12))
  (fp_line (start 0.25 1.46) (end 7.37 1.46) (layer F.SilkS) (width 0.12))
  (fp_line (start 0 1.99) (end 0.25 1.46) (layer F.SilkS) (width 0.12))
  (fp_line (start 7.62 1.99) (end 7.62 2.99) (layer F.SilkS) (width 0.12))
  (fp_line (start 0 1.99) (end 7.62 1.99) (layer F.SilkS) (width 0.12))
  (fp_line (start 0 2.99) (end 0 1.99) (layer F.SilkS) (width 0.12))
  (fp_line (start -1.67 -2) (end -1.67 2) (layer F.SilkS) (width 0.12))
  (fp_line (start 9 -3.03) (end -1.38 -3.03) (layer F.SilkS) (width 0.12))
  (fp_line (start 9 2.99) (end 9 -3.03) (layer F.SilkS) (width 0.12))
  (fp_line (start -1.38 2.99) (end 9 2.99) (layer F.SilkS) (width 0.12))
  (fp_line (start -1.38 -3.03) (end -1.38 2.99) (layer F.SilkS) (width 0.12))
  (pad 4 thru_hole oval (at 7.62 0 90) (size 1.74 2.2) (drill 1.2) (layers *.Cu *.Mask) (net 10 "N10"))
  (pad 3 thru_hole oval (at 5.08 0 90) (size 1.74 2.2) (drill 1.2) (layers *.Cu *.Mask) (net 2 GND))
  (pad 2 thru_hole oval (at 2.54 0 90) (size 1.74 2.2) (drill 1.2) (layers *.Cu *.Mask) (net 9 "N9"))
  (pad 1 thru_hole roundrect (at 0 0 90) (size 1.74 2.2) (drill 1.2) (layers *.Cu *.Mask) (roundrect_rratio 0.143678) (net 4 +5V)))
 (gr_line (start 114.6 81.2) (end 114.6 58.2) (layer Edge.Cuts) (width 0.05))
 (gr_line (start 136.6 81.2) (end 114.6 81.2) (layer Edge.Cuts) (width 0.05))
 (gr_line (start 136.6 58.2) (end 136.6 81.2) (layer Edge.Cuts) (width 0.05))
 (gr_line (start 114.6 58.2) (end 136.6 58.2) (layer Edge.Cuts) (width 0.05))
 (segment (start 123.345 74.12) (end 124.2 74.975) (width 1.4) (layer B.Cu) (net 2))
 (segment (start 118.2 74.12) (end 123.345 74.12) (width 1.4) (layer B.Cu) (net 2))
 (segment (start 123.345 62.72) (end 124.2 63.575) (width 1.4) (layer B.Cu) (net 2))
 (segment (start 118.2 62.72) (end 123.345 62.72) (width 1.4) (layer B.Cu) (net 2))
 (segment (start 135.5 74.12) (end 133 74.12) (width 1.4) (layer B.Cu) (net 2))
 (segment (start 135.67499 73.94501) (end 135.5 74.12) (width 1.4) (layer B.Cu) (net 2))
 (segment (start 135.67499 62.89499) (end 135.67499 73.94501) (width 1.4) (layer B.Cu) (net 2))
 (segment (start 133 62.72) (end 135.5 62.72) (width 1.4) (layer B.Cu) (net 2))
 (segment (start 135.5 62.72) (end 135.67499 62.89499) (width 1.4) (layer B.Cu) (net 2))
 (segment (start 118.2 67.8) (end 133 67.8) (width 1.4) (layer B.Cu) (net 4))
 (segment (start 118.2 79.2) (end 133 79.2) (width 1.4) (layer B.Cu) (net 4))
 (segment (start 117 67.8) (end 115.8 69) (width 1.4) (layer B.Cu) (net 4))
 (segment (start 118.2 67.8) (end 117 67.8) (width 1.4) (layer B.Cu) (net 4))
 (segment (start 117 79.2) (end 118.2 79.2) (width 1.4) (layer B.Cu) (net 4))
 (segment (start 115.8 78) (end 117 79.2) (width 1.4) (layer B.Cu) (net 4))
 (segment (start 115.8 69) (end 115.8 78) (width 1.4) (layer B.Cu) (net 4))
 (segment (start 118.605 59.775) (end 118.2 60.18) (width 1.4) (layer B.Cu) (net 5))
 (segment (start 124.2 59.775) (end 118.605 59.775) (width 1.4) (layer B.Cu) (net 5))
 (segment (start 126.55 59.775) (end 126.575 59.8) (width 1) (layer B.Cu) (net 5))
 (segment (start 124.2 59.775) (end 126.55 59.775) (width 1) (layer B.Cu) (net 5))
 (segment (start 132.62 59.8) (end 133 60.18) (width 1.4) (layer B.Cu) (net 10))
 (segment (start 128.625 59.8) (end 132.62 59.8) (width 1.4) (layer B.Cu) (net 10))
 (segment (start 118.605 71.175) (end 118.2 71.58) (width 1.4) (layer B.Cu) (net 1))
 (segment (start 124.2 71.175) (end 118.605 71.175) (width 1.4) (layer B.Cu) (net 1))
 (segment (start 132.62 71.2) (end 133 71.58) (width 1.4) (layer B.Cu) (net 8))
 (segment (start 128.625 71.2) (end 132.62 71.2) (width 1.4) (layer B.Cu) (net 8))
 (segment (start 118.565 77.025) (end 118.2 76.66) (width 1.4) (layer B.Cu) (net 3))
 (segment (start 124.2 77.025) (end 118.565 77.025) (width 1.4) (layer B.Cu) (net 3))
 (segment (start 132.66 77) (end 133 76.66) (width 1.4) (layer B.Cu) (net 7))
 (segment (start 128.625 77) (end 132.66 77) (width 1.4) (layer B.Cu) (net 7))
 (segment (start 128.965 65.26) (end 128.625 65.6) (width 1.4) (layer B.Cu) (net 9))
 (segment (start 133 65.26) (end 128.965 65.26) (width 1.4) (layer B.Cu) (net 9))
 (segment (start 118.565 65.625) (end 118.2 65.26) (width 1.4) (layer B.Cu) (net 6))
 (segment (start 124.2 65.625) (end 118.565 65.625) (width 1.4) (layer B.Cu) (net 6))
 (segment (start 126.55 65.625) (end 126.575 65.6) (width 1) (layer B.Cu) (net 6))
 (segment (start 124.2 65.625) (end 126.55 65.625) (width 1) (layer B.Cu) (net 6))
 (segment (start 126.55 71.175) (end 126.575 71.2) (width 1) (layer B.Cu) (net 1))
 (segment (start 124.2 71.175) (end 126.55 71.175) (width 1) (layer B.Cu) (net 1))
 (segment (start 126.55 77.025) (end 126.575 77) (width 1) (layer B.Cu) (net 3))
 (segment (start 124.2 77.025) (end 126.55 77.025) (width 1) (layer B.Cu) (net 3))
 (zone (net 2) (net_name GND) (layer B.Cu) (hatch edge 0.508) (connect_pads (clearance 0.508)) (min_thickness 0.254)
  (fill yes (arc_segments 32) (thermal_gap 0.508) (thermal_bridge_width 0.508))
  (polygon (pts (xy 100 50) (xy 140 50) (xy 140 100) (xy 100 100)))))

